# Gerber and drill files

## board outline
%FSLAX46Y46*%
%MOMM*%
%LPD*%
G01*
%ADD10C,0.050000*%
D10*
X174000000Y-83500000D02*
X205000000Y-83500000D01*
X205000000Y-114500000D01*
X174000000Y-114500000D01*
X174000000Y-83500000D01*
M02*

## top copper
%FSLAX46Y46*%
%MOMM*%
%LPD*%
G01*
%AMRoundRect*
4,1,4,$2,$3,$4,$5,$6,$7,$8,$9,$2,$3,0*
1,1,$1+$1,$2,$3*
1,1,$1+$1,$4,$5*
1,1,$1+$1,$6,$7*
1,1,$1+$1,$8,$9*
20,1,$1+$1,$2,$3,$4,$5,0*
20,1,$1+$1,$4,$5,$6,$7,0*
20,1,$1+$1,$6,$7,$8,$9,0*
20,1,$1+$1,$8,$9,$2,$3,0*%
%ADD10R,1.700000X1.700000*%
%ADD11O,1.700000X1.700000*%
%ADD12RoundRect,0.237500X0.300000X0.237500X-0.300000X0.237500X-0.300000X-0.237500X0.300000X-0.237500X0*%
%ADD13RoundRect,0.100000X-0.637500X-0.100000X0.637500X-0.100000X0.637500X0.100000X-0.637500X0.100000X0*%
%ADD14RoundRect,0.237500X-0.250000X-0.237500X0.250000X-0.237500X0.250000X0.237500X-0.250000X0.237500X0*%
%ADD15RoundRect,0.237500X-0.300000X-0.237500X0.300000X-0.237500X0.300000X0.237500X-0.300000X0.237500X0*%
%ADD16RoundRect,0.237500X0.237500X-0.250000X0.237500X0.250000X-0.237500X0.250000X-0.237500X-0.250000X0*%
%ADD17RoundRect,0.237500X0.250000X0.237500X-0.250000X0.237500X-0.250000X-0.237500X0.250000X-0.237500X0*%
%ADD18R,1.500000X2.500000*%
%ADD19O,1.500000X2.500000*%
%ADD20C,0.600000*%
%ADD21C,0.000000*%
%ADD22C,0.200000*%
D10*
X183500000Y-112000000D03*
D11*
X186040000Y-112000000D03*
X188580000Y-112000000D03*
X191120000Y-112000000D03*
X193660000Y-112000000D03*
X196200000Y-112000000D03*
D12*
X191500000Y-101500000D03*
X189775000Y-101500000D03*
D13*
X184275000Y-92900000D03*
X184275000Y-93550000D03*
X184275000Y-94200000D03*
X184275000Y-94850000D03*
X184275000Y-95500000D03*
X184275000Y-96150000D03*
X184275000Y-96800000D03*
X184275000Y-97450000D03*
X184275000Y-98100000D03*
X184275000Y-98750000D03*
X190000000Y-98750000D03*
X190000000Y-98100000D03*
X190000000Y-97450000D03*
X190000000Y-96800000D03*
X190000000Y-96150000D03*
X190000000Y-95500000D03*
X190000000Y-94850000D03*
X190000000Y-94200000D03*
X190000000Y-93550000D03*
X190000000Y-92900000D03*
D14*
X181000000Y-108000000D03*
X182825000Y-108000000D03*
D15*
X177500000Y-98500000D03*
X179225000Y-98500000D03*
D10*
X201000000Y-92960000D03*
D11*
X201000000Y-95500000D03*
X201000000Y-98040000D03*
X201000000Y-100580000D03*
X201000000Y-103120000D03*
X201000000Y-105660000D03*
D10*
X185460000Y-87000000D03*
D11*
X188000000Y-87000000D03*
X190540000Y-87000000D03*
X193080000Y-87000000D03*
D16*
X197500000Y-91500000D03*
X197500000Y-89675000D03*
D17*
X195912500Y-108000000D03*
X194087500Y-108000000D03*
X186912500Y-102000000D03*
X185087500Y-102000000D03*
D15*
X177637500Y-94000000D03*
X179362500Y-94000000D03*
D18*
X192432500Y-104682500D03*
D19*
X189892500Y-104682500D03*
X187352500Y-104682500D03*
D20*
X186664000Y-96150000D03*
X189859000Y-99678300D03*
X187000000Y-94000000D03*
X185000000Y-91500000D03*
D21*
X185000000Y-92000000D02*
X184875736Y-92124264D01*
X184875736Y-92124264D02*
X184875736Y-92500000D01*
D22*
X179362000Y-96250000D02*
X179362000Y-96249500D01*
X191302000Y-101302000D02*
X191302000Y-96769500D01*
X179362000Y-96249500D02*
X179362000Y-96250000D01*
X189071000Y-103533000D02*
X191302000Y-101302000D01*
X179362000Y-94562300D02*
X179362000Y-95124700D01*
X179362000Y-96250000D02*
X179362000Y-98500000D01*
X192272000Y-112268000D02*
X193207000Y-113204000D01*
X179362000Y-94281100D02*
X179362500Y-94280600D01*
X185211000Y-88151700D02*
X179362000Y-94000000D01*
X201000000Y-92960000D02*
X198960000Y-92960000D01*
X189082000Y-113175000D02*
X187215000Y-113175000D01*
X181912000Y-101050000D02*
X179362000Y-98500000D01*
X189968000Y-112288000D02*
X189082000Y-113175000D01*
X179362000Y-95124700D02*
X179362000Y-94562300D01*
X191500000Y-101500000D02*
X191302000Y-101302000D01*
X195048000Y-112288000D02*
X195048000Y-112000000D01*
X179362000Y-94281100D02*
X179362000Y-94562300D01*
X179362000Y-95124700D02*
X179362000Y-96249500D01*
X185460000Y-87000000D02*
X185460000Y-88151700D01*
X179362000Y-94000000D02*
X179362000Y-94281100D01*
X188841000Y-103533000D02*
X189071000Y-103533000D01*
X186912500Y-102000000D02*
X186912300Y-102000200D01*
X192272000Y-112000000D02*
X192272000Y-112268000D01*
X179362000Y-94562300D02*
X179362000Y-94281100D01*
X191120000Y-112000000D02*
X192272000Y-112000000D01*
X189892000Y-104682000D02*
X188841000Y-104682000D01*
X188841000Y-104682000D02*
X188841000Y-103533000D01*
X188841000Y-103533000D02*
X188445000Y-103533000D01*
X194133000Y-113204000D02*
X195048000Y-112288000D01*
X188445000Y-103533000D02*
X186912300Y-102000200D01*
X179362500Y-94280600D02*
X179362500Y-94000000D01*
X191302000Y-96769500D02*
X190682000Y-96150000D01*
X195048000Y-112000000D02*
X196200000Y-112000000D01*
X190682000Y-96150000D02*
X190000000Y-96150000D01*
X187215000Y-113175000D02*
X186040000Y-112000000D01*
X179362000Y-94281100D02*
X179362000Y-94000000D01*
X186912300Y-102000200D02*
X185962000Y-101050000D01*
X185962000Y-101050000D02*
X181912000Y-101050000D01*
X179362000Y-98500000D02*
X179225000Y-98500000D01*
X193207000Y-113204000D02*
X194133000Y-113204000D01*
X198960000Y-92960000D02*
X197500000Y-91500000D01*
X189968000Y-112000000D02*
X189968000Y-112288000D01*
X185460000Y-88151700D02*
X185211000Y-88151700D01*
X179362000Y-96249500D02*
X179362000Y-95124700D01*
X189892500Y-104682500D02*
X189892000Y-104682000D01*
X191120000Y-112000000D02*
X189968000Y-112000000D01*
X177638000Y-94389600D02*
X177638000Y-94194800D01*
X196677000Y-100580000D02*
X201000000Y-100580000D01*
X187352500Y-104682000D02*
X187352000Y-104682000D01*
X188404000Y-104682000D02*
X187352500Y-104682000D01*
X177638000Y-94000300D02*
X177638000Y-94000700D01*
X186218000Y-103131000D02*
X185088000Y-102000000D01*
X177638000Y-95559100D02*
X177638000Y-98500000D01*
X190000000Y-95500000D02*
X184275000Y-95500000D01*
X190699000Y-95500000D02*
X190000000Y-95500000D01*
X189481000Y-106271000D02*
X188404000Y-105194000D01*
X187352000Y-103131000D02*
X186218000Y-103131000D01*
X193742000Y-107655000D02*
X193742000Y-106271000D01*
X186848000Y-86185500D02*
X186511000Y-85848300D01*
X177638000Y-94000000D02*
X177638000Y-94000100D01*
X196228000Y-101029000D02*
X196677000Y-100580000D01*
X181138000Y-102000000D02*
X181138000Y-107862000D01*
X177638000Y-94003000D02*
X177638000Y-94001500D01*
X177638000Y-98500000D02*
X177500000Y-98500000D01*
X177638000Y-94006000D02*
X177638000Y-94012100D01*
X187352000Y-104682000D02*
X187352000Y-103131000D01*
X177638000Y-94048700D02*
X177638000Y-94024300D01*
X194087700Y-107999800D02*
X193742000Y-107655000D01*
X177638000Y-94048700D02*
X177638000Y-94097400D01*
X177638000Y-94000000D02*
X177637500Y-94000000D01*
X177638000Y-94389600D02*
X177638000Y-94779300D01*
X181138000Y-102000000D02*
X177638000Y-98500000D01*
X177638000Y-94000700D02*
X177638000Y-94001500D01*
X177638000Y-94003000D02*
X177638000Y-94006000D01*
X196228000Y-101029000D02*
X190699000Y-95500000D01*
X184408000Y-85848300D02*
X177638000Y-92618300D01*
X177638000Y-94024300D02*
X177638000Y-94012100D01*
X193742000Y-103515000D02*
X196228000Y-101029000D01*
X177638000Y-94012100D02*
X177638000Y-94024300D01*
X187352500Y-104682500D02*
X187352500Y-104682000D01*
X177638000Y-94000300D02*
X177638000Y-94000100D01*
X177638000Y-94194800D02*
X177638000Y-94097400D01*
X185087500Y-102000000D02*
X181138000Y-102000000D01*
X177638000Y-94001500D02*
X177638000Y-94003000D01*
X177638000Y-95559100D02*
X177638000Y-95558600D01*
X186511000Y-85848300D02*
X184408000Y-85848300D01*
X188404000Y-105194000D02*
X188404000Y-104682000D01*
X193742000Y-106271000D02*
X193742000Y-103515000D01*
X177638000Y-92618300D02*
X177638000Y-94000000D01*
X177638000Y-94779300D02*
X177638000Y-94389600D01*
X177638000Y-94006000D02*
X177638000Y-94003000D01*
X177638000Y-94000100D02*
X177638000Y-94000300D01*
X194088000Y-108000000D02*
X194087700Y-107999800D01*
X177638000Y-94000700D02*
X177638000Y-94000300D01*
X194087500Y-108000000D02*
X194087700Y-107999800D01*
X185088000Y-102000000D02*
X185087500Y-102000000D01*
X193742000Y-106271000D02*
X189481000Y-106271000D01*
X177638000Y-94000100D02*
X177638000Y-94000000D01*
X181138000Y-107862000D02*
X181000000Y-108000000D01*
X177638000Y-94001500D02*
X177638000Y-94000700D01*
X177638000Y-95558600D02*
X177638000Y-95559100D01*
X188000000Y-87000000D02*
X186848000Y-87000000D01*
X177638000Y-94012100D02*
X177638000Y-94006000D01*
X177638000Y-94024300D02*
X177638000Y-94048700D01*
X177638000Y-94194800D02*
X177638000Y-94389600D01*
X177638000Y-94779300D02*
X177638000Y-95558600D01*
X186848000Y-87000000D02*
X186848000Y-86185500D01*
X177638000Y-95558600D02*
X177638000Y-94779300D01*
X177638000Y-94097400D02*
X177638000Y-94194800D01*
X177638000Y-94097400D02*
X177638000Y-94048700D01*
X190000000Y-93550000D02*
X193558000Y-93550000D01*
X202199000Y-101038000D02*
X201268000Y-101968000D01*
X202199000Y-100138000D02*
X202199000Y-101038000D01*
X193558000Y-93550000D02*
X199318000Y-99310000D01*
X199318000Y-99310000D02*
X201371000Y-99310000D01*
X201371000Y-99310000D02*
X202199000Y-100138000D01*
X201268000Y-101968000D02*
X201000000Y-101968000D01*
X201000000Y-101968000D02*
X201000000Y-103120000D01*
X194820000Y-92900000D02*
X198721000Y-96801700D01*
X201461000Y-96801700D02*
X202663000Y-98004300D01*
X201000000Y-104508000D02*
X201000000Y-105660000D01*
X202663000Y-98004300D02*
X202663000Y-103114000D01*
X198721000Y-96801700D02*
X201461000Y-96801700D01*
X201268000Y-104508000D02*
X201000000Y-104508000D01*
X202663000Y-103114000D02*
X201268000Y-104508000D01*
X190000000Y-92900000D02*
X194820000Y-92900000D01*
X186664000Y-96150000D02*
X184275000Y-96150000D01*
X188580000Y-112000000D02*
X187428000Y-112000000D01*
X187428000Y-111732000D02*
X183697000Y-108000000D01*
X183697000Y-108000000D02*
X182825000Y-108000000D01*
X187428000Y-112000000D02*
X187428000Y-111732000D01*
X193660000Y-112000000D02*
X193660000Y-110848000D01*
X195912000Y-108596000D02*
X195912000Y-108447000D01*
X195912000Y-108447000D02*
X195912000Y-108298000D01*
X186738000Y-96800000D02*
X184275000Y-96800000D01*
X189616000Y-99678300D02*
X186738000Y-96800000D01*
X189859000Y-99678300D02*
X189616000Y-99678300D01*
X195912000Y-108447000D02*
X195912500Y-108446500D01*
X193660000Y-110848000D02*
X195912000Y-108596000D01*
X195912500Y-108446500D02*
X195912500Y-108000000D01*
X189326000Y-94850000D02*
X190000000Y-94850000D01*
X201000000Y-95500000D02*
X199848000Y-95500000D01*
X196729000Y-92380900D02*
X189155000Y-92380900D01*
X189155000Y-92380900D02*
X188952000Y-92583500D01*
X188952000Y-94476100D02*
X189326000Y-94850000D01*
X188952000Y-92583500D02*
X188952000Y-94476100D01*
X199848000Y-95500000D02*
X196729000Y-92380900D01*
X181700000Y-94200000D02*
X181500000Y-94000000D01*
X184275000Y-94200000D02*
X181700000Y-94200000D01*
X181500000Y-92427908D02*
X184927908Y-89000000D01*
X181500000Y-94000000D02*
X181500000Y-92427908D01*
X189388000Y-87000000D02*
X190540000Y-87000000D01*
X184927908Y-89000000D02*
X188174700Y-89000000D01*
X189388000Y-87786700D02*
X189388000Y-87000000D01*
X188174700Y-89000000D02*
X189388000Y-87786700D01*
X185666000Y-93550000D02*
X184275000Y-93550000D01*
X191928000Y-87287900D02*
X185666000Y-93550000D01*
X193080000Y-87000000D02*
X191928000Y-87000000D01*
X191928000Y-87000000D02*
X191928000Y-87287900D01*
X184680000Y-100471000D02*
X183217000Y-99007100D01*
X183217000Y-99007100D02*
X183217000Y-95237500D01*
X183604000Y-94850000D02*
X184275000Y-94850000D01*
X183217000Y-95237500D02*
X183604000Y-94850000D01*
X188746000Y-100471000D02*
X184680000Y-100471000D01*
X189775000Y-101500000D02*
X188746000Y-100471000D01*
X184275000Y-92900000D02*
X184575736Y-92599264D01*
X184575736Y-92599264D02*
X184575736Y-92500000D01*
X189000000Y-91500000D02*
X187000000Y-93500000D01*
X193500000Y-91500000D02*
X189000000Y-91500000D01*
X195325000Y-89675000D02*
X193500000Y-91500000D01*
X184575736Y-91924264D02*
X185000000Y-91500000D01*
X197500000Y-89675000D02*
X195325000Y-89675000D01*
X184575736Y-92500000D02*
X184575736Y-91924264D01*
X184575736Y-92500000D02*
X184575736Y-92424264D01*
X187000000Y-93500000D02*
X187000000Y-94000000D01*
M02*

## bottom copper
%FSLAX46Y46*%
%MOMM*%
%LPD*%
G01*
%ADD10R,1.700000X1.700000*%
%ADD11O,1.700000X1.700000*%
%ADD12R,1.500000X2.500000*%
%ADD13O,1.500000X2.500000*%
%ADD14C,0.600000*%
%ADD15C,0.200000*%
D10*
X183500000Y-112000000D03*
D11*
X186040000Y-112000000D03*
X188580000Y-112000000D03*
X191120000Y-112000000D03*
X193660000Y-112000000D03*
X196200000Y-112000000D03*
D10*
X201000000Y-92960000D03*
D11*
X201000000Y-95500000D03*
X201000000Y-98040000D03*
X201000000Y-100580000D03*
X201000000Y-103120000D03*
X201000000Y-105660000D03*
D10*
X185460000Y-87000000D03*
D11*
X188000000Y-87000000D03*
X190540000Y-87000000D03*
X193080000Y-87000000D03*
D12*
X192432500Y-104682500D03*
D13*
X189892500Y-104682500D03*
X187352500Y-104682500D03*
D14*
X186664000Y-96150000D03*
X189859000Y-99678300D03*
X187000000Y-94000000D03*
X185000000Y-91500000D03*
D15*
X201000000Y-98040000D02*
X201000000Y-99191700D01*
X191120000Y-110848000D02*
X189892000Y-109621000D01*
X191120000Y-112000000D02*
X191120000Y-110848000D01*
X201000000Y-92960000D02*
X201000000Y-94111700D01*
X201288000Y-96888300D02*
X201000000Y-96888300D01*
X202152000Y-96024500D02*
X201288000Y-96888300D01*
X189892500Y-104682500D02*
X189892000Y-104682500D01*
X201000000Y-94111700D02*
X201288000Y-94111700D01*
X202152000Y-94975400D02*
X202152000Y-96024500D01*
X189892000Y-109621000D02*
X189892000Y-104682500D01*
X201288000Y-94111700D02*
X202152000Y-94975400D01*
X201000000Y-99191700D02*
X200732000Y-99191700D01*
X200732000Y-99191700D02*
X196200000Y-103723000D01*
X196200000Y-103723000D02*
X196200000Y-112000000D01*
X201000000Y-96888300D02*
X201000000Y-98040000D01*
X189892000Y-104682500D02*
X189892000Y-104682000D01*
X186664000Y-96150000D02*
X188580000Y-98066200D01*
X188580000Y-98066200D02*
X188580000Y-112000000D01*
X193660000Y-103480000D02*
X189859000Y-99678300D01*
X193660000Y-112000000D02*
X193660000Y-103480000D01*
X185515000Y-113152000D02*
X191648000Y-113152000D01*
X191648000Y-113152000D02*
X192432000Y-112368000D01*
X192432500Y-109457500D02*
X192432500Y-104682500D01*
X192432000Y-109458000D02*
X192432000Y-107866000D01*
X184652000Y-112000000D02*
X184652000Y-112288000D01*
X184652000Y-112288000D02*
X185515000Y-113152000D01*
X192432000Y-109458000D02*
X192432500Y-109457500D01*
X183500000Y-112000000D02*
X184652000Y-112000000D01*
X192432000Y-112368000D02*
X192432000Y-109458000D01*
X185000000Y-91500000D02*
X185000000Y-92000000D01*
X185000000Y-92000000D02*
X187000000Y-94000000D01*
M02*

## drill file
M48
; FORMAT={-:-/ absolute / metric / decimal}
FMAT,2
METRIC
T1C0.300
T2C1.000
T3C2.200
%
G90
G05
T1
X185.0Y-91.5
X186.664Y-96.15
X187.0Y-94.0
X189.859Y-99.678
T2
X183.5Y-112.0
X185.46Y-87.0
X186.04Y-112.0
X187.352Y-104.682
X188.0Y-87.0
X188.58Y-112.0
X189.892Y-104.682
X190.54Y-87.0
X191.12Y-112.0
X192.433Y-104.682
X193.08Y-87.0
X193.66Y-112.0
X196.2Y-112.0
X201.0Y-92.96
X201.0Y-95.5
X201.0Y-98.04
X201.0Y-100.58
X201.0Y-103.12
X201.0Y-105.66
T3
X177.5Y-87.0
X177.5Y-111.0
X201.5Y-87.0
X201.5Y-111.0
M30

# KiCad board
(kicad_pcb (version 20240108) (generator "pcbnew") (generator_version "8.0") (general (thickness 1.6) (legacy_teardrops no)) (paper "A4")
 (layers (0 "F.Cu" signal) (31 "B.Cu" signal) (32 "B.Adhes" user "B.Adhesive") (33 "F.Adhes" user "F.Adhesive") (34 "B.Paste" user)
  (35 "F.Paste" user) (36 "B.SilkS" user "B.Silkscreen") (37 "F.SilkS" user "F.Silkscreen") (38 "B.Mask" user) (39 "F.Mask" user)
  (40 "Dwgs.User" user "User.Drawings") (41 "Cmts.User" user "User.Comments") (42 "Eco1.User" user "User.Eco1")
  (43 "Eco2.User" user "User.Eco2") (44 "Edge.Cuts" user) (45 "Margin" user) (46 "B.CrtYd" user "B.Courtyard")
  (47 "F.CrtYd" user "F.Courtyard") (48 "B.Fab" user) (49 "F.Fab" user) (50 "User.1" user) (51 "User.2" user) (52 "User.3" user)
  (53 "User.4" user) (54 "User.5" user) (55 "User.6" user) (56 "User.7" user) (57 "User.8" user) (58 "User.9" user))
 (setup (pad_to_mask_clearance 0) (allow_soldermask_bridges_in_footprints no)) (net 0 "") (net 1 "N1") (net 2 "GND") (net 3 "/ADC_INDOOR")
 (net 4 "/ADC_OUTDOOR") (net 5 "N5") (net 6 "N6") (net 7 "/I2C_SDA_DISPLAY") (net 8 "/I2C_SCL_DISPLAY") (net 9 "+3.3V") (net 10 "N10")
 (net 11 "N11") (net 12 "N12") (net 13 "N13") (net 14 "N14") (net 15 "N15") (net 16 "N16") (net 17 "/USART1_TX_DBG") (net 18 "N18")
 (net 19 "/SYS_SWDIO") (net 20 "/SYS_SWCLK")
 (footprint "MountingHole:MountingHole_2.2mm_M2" (layer "F.Cu") (at 201.5 111)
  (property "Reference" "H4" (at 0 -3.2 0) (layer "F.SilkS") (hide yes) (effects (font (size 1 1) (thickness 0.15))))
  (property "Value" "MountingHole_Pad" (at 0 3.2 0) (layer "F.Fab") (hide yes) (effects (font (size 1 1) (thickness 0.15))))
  (pad "" np_thru_hole circle (at 0 0) (size 2.2 2.2) (drill 2.2) (layers "*.Cu" "*.Mask")))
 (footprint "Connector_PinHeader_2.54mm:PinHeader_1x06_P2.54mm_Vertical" (layer "F.Cu") (at 183.5 112 90)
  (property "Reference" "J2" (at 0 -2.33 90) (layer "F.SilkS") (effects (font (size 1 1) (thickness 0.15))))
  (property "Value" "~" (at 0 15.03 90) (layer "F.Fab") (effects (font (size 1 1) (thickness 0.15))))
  (pad "1" thru_hole rect (at 0 0 90) (size 1.7 1.7) (drill 1) (layers "*.Cu" "*.Mask") (remove_unused_layers no) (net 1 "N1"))
  (pad "2" thru_hole oval (at 0 2.54 90) (size 1.7 1.7) (drill 1) (layers "*.Cu" "*.Mask") (remove_unused_layers no) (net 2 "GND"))
  (pad "3" thru_hole oval (at 0 5.08 90) (size 1.7 1.7) (drill 1) (layers "*.Cu" "*.Mask") (remove_unused_layers no) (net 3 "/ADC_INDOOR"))
  (pad "4" thru_hole oval (at 0 7.62 90) (size 1.7 1.7) (drill 1) (layers "*.Cu" "*.Mask") (remove_unused_layers no) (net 2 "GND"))
  (pad "5" thru_hole oval (at 0 10.16 90) (size 1.7 1.7) (drill 1) (layers "*.Cu" "*.Mask") (remove_unused_layers no) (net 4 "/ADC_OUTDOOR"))
  (pad "6" thru_hole oval (at 0 12.7 90) (size 1.7 1.7) (drill 1) (layers "*.Cu" "*.Mask") (remove_unused_layers no) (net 2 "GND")))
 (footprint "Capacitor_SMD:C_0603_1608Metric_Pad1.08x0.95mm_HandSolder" (layer "F.Cu") (at 190.6375 101.5 180)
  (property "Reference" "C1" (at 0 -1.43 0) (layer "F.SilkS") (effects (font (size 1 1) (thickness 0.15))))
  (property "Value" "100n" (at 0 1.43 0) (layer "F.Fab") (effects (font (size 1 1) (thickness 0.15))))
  (pad "1" smd roundrect (at -0.8625 0 180) (size 1.075 0.95) (layers "F.Cu" "F.Paste" "F.Mask") (roundrect_rratio 0.25) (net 2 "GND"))
  (pad "2" smd roundrect (at 0.8625 0 180) (size 1.075 0.95) (layers "F.Cu" "F.Paste" "F.Mask") (roundrect_rratio 0.25) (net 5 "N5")))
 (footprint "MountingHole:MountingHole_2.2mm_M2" (layer "F.Cu") (at 201.5 87)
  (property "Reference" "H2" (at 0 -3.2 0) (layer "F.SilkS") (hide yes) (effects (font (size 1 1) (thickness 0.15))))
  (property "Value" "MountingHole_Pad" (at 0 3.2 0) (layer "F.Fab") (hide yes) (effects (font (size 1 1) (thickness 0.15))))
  (pad "" np_thru_hole circle (at 0 0) (size 2.2 2.2) (drill 2.2) (layers "*.Cu" "*.Mask")))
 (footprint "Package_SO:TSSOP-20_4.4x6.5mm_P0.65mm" (layer "F.Cu") (at 187.1375 95.825)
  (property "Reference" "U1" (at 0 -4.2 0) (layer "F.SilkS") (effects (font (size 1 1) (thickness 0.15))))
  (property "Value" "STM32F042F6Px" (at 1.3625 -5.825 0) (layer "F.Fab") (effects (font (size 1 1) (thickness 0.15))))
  (pad "1" smd roundrect (at -2.8625 -2.925) (size 1.475 0.4) (layers "F.Cu" "F.Paste" "F.Mask") (roundrect_rratio 0.25) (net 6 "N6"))
  (pad "2" smd roundrect (at -2.8625 -2.275) (size 1.475 0.4) (layers "F.Cu" "F.Paste" "F.Mask") (roundrect_rratio 0.25)
   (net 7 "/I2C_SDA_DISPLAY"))
  (pad "3" smd roundrect (at -2.8625 -1.625) (size 1.475 0.4) (layers "F.Cu" "F.Paste" "F.Mask") (roundrect_rratio 0.25)
   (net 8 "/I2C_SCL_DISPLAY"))
  (pad "4" smd roundrect (at -2.8625 -0.975) (size 1.475 0.4) (layers "F.Cu" "F.Paste" "F.Mask") (roundrect_rratio 0.25) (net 5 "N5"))
  (pad "5" smd roundrect (at -2.8625 -0.325) (size 1.475 0.4) (layers "F.Cu" "F.Paste" "F.Mask") (roundrect_rratio 0.25) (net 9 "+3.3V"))
  (pad "6" smd roundrect (at -2.8625 0.325) (size 1.475 0.4) (layers "F.Cu" "F.Paste" "F.Mask") (roundrect_rratio 0.25)
   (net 3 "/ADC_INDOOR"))
  (pad "7" smd roundrect (at -2.8625 0.975) (size 1.475 0.4) (layers "F.Cu" "F.Paste" "F.Mask") (roundrect_rratio 0.25)
   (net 4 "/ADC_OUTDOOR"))
  (pad "8" smd roundrect (at -2.8625 1.625) (size 1.475 0.4) (layers "F.Cu" "F.Paste" "F.Mask") (roundrect_rratio 0.25) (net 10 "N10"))
  (pad "9" smd roundrect (at -2.8625 2.275) (size 1.475 0.4) (layers "F.Cu" "F.Paste" "F.Mask") (roundrect_rratio 0.25) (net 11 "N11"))
  (pad "10" smd roundrect (at -2.8625 2.925) (size 1.475 0.4) (layers "F.Cu" "F.Paste" "F.Mask") (roundrect_rratio 0.25) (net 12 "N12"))
  (pad "11" smd roundrect (at 2.8625 2.925) (size 1.475 0.4) (layers "F.Cu" "F.Paste" "F.Mask") (roundrect_rratio 0.25) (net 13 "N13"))
  (pad "12" smd roundrect (at 2.8625 2.275) (size 1.475 0.4) (layers "F.Cu" "F.Paste" "F.Mask") (roundrect_rratio 0.25) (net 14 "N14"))
  (pad "13" smd roundrect (at 2.8625 1.625) (size 1.475 0.4) (layers "F.Cu" "F.Paste" "F.Mask") (roundrect_rratio 0.25) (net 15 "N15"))
  (pad "14" smd roundrect (at 2.8625 0.975) (size 1.475 0.4) (layers "F.Cu" "F.Paste" "F.Mask") (roundrect_rratio 0.25) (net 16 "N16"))
  (pad "15" smd roundrect (at 2.8625 0.325) (size 1.475 0.4) (layers "F.Cu" "F.Paste" "F.Mask") (roundrect_rratio 0.25) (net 2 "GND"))
  (pad "16" smd roundrect (at 2.8625 -0.325) (size 1.475 0.4) (layers "F.Cu" "F.Paste" "F.Mask") (roundrect_rratio 0.25) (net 9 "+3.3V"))
  (pad "17" smd roundrect (at 2.8625 -0.975) (size 1.475 0.4) (layers "F.Cu" "F.Paste" "F.Mask") (roundrect_rratio 0.25)
   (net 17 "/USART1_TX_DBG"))
  (pad "18" smd roundrect (at 2.8625 -1.625) (size 1.475 0.4) (layers "F.Cu" "F.Paste" "F.Mask") (roundrect_rratio 0.25) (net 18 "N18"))
  (pad "19" smd roundrect (at 2.8625 -2.275) (size 1.475 0.4) (layers "F.Cu" "F.Paste" "F.Mask") (roundrect_rratio 0.25)
   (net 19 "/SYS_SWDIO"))
  (pad "20" smd roundrect (at 2.8625 -2.925) (size 1.475 0.4) (layers "F.Cu" "F.Paste" "F.Mask") (roundrect_rratio 0.25)
   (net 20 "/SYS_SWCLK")))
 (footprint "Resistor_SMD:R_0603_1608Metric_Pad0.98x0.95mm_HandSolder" (layer "F.Cu") (at 181.9125 108)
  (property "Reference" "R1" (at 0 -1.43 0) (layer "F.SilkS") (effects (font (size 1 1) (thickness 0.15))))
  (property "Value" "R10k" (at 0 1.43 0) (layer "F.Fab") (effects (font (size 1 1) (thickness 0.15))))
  (pad "1" smd roundrect (at -0.9125 0) (size 0.975 0.95) (layers "F.Cu" "F.Paste" "F.Mask") (roundrect_rratio 0.25) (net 9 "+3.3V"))
  (pad "2" smd roundrect (at 0.9125 0) (size 0.975 0.95) (layers "F.Cu" "F.Paste" "F.Mask") (roundrect_rratio 0.25) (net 3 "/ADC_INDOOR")))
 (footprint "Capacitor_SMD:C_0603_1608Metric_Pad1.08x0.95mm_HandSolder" (layer "F.Cu") (at 178.3625 98.5)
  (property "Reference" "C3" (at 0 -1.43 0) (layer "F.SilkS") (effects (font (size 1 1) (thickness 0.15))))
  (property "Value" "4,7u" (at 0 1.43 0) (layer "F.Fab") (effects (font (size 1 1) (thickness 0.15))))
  (pad "1" smd roundrect (at -0.8625 0) (size 1.075 0.95) (layers "F.Cu" "F.Paste" "F.Mask") (roundrect_rratio 0.25) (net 9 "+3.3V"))
  (pad "2" smd roundrect (at 0.8625 0) (size 1.075 0.95) (layers "F.Cu" "F.Paste" "F.Mask") (roundrect_rratio 0.25) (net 2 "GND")))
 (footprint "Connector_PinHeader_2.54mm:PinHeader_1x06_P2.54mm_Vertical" (layer "F.Cu") (at 201 92.96)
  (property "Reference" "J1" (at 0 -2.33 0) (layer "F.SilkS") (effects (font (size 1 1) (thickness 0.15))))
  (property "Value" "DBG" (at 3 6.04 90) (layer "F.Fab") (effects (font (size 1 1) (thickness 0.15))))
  (pad "1" thru_hole rect (at 0 0) (size 1.7 1.7) (drill 1) (layers "*.Cu" "*.Mask") (remove_unused_layers no) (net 2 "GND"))
  (pad "2" thru_hole oval (at 0 2.54) (size 1.7 1.7) (drill 1) (layers "*.Cu" "*.Mask") (remove_unused_layers no) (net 17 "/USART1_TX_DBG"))
  (pad "3" thru_hole oval (at 0 5.08) (size 1.7 1.7) (drill 1) (layers "*.Cu" "*.Mask") (remove_unused_layers no) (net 2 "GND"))
  (pad "4" thru_hole oval (at 0 7.62) (size 1.7 1.7) (drill 1) (layers "*.Cu" "*.Mask") (remove_unused_layers no) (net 9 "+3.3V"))
  (pad "5" thru_hole oval (at 0 10.16) (size 1.7 1.7) (drill 1) (layers "*.Cu" "*.Mask") (remove_unused_layers no) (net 19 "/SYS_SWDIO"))
  (pad "6" thru_hole oval (at 0 12.7) (size 1.7 1.7) (drill 1) (layers "*.Cu" "*.Mask") (remove_unused_layers no) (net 20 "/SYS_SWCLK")))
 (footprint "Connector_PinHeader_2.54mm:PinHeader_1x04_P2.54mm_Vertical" (layer "F.Cu") (at 185.46 87 90)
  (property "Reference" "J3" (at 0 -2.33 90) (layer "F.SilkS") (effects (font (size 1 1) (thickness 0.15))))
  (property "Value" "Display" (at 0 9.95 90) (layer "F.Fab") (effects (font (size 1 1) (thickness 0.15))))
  (pad "1" thru_hole rect (at 0 0 90) (size 1.7 1.7) (drill 1) (layers "*.Cu" "*.Mask") (remove_unused_layers no) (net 2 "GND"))
  (pad "2" thru_hole oval (at 0 2.54 90) (size 1.7 1.7) (drill 1) (layers "*.Cu" "*.Mask") (remove_unused_layers no) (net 9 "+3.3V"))
  (pad "3" thru_hole oval (at 0 5.08 90) (size 1.7 1.7) (drill 1) (layers "*.Cu" "*.Mask") (remove_unused_layers no)
   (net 8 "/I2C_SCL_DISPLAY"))
  (pad "4" thru_hole oval (at 0 7.62 90) (size 1.7 1.7) (drill 1) (layers "*.Cu" "*.Mask") (remove_unused_layers no)
   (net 7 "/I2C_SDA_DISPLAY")))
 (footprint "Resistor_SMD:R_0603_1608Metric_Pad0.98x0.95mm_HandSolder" (layer "F.Cu") (at 197.5 90.5875 90)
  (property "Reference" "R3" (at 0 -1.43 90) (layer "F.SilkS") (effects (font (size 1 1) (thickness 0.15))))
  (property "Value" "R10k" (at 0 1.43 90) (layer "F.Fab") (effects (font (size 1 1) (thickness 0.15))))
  (pad "1" smd roundrect (at -0.9125 0 90) (size 0.975 0.95) (layers "F.Cu" "F.Paste" "F.Mask") (roundrect_rratio 0.25) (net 2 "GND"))
  (pad "2" smd roundrect (at 0.9125 0 90) (size 0.975 0.95) (layers "F.Cu" "F.Paste" "F.Mask") (roundrect_rratio 0.25) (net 6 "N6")))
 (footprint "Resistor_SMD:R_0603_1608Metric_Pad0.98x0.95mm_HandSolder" (layer "F.Cu") (at 195 108 180)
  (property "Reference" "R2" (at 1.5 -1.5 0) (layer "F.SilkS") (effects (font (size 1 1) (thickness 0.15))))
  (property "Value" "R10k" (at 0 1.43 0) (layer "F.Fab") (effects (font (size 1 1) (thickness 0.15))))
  (pad "1" smd roundrect (at -0.9125 0 180) (size 0.975 0.95) (layers "F.Cu" "F.Paste" "F.Mask") (roundrect_rratio 0.25)
   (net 4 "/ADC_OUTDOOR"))
  (pad "2" smd roundrect (at 0.9125 0 180) (size 0.975 0.95) (layers "F.Cu" "F.Paste" "F.Mask") (roundrect_rratio 0.25) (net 9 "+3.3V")))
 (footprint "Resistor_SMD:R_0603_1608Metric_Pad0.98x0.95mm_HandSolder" (layer "F.Cu") (at 186 102 180)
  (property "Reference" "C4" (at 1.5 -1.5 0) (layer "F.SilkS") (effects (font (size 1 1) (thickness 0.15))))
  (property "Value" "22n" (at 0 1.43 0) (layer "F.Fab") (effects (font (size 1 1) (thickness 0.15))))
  (pad "1" smd roundrect (at -0.9125 0 180) (size 0.975 0.95) (layers "F.Cu" "F.Paste" "F.Mask") (roundrect_rratio 0.25) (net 2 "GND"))
  (pad "2" smd roundrect (at 0.9125 0 180) (size 0.975 0.95) (layers "F.Cu" "F.Paste" "F.Mask") (roundrect_rratio 0.25) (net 9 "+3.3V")))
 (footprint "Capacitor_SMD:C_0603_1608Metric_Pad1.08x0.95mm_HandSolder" (layer "F.Cu") (at 178.5 94)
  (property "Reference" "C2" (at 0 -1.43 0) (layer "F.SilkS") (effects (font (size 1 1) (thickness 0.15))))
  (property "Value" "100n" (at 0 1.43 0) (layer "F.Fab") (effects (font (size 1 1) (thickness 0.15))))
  (pad "1" smd roundrect (at -0.8625 0) (size 1.075 0.95) (layers "F.Cu" "F.Paste" "F.Mask") (roundrect_rratio 0.25) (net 9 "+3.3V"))
  (pad "2" smd roundrect (at 0.8625 0) (size 1.075 0.95) (layers "F.Cu" "F.Paste" "F.Mask") (roundrect_rratio 0.25) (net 2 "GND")))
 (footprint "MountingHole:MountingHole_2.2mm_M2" (layer "F.Cu") (at 177.5 87)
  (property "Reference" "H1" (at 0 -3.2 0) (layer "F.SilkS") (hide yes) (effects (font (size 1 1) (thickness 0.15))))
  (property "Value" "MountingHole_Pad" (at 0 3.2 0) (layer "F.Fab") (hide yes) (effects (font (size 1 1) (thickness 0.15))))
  (pad "" np_thru_hole circle (at 0 0) (size 2.2 2.2) (drill 2.2) (layers "*.Cu" "*.Mask")))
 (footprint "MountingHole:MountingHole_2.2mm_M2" (layer "F.Cu") (at 177.5 111)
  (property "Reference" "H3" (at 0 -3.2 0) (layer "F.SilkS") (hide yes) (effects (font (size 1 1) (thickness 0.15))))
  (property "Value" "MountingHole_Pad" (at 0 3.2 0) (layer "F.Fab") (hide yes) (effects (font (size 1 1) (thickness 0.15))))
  (pad "" np_thru_hole circle (at 0 0) (size 2.2 2.2) (drill 2.2) (layers "*.Cu" "*.Mask")))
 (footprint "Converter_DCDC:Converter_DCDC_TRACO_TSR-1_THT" (layer "B.Cu") (at 192.4325 104.6825 180)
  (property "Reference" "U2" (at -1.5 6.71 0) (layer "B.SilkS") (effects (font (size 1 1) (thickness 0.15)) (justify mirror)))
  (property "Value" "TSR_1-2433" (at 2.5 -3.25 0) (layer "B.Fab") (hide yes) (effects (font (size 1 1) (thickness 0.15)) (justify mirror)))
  (pad "1" thru_hole rect (at 0 0 180) (size 1.5 2.5) (drill 1) (layers "*.Cu" "*.Mask") (remove_unused_layers no) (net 1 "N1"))
  (pad "2" thru_hole oval (at 2.54 0 180) (size 1.5 2.5) (drill 1) (layers "*.Cu" "*.Mask") (remove_unused_layers no) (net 2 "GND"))
  (pad "3" thru_hole oval (at 5.08 0 180) (size 1.5 2.5) (drill 1) (layers "*.Cu" "*.Mask") (remove_unused_layers no) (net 9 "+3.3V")))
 (gr_rect (start 174 83.5) (end 205 114.5) (stroke (width 0.05) (type default)) (fill none) (layer "Edge.Cuts"))
 (segment (start 185 92) (end 184.875736 92.124264) (width 0) (layer "F.Cu") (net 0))
 (segment (start 184.875736 92.124264) (end 184.875736 92.5) (width 0) (layer "F.Cu") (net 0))
 (segment (start 179.362 96.25) (end 179.362 96.2495) (width 0.2) (layer "F.Cu") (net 2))
 (segment (start 191.302 101.302) (end 191.302 96.7695) (width 0.2) (layer "F.Cu") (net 2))
 (segment (start 179.362 96.2495) (end 179.362 96.25) (width 0.2) (layer "F.Cu") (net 2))
 (segment (start 189.071 103.533) (end 191.302 101.302) (width 0.2) (layer "F.Cu") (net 2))
 (segment (start 179.362 94.5623) (end 179.362 95.1247) (width 0.2) (layer "F.Cu") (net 2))
 (segment (start 179.362 96.25) (end 179.362 98.5) (width 0.2) (layer "F.Cu") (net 2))
 (segment (start 192.272 112.268) (end 193.207 113.204) (width 0.2) (layer "F.Cu") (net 2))
 (segment (start 179.362 94.2811) (end 179.3625 94.2806) (width 0.2) (layer "F.Cu") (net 2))
 (segment (start 185.211 88.1517) (end 179.362 94) (width 0.2) (layer "F.Cu") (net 2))
 (segment (start 201 92.96) (end 198.96 92.96) (width 0.2) (layer "F.Cu") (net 2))
 (segment (start 189.082 113.175) (end 187.215 113.175) (width 0.2) (layer "F.Cu") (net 2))
 (segment (start 181.912 101.05) (end 179.362 98.5) (width 0.2) (layer "F.Cu") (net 2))
 (segment (start 189.968 112.288) (end 189.082 113.175) (width 0.2) (layer "F.Cu") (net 2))
 (segment (start 179.362 95.1247) (end 179.362 94.5623) (width 0.2) (layer "F.Cu") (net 2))
 (segment (start 191.5 101.5) (end 191.302 101.302) (width 0.2) (layer "F.Cu") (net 2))
 (segment (start 195.048 112.288) (end 195.048 112) (width 0.2) (layer "F.Cu") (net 2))
 (segment (start 179.362 94.2811) (end 179.362 94.5623) (width 0.2) (layer "F.Cu") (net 2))
 (segment (start 179.362 95.1247) (end 179.362 96.2495) (width 0.2) (layer "F.Cu") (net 2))
 (segment (start 185.46 87) (end 185.46 88.1517) (width 0.2) (layer "F.Cu") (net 2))
 (segment (start 179.362 94) (end 179.362 94.2811) (width 0.2) (layer "F.Cu") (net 2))
 (segment (start 188.841 103.533) (end 189.071 103.533) (width 0.2) (layer "F.Cu") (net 2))
 (segment (start 186.9125 102) (end 186.9123 102.0002) (width 0.2) (layer "F.Cu") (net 2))
 (segment (start 192.272 112) (end 192.272 112.268) (width 0.2) (layer "F.Cu") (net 2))
 (segment (start 179.362 94.5623) (end 179.362 94.2811) (width 0.2) (layer "F.Cu") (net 2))
 (segment (start 191.12 112) (end 192.272 112) (width 0.2) (layer "F.Cu") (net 2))
 (segment (start 189.892 104.682) (end 188.841 104.682) (width 0.2) (layer "F.Cu") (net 2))
 (segment (start 188.841 104.682) (end 188.841 103.533) (width 0.2) (layer "F.Cu") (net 2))
 (segment (start 188.841 103.533) (end 188.445 103.533) (width 0.2) (layer "F.Cu") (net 2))
 (segment (start 194.133 113.204) (end 195.048 112.288) (width 0.2) (layer "F.Cu") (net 2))
 (segment (start 188.445 103.533) (end 186.9123 102.0002) (width 0.2) (layer "F.Cu") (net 2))
 (segment (start 179.3625 94.2806) (end 179.3625 94) (width 0.2) (layer "F.Cu") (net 2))
 (segment (start 191.302 96.7695) (end 190.682 96.15) (width 0.2) (layer "F.Cu") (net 2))
 (segment (start 195.048 112) (end 196.2 112) (width 0.2) (layer "F.Cu") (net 2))
 (segment (start 190.682 96.15) (end 190 96.15) (width 0.2) (layer "F.Cu") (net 2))
 (segment (start 187.215 113.175) (end 186.04 112) (width 0.2) (layer "F.Cu") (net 2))
 (segment (start 179.362 94.2811) (end 179.362 94) (width 0.2) (layer "F.Cu") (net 2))
 (segment (start 186.9123 102.0002) (end 185.962 101.05) (width 0.2) (layer "F.Cu") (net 2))
 (segment (start 185.962 101.05) (end 181.912 101.05) (width 0.2) (layer "F.Cu") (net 2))
 (segment (start 179.362 98.5) (end 179.225 98.5) (width 0.2) (layer "F.Cu") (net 2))
 (segment (start 193.207 113.204) (end 194.133 113.204) (width 0.2) (layer "F.Cu") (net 2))
 (segment (start 198.96 92.96) (end 197.5 91.5) (width 0.2) (layer "F.Cu") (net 2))
 (segment (start 189.968 112) (end 189.968 112.288) (width 0.2) (layer "F.Cu") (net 2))
 (segment (start 185.46 88.1517) (end 185.211 88.1517) (width 0.2) (layer "F.Cu") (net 2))
 (segment (start 179.362 96.2495) (end 179.362 95.1247) (width 0.2) (layer "F.Cu") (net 2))
 (segment (start 189.8925 104.6825) (end 189.892 104.682) (width 0.2) (layer "F.Cu") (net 2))
 (segment (start 191.12 112) (end 189.968 112) (width 0.2) (layer "F.Cu") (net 2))
 (segment (start 201 98.04) (end 201 99.1917) (width 0.2) (layer "B.Cu") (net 2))
 (segment (start 191.12 110.848) (end 189.892 109.621) (width 0.2) (layer "B.Cu") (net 2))
 (segment (start 191.12 112) (end 191.12 110.848) (width 0.2) (layer "B.Cu") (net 2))
 (segment (start 201 92.96) (end 201 94.1117) (width 0.2) (layer "B.Cu") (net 2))
 (segment (start 201.288 96.8883) (end 201 96.8883) (width 0.2) (layer "B.Cu") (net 2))
 (segment (start 202.152 96.0245) (end 201.288 96.8883) (width 0.2) (layer "B.Cu") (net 2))
 (segment (start 189.8925 104.6825) (end 189.892 104.6825) (width 0.2) (layer "B.Cu") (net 2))
 (segment (start 201 94.1117) (end 201.288 94.1117) (width 0.2) (layer "B.Cu") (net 2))
 (segment (start 202.152 94.9754) (end 202.152 96.0245) (width 0.2) (layer "B.Cu") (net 2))
 (segment (start 189.892 109.621) (end 189.892 104.6825) (width 0.2) (layer "B.Cu") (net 2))
 (segment (start 201.288 94.1117) (end 202.152 94.9754) (width 0.2) (layer "B.Cu") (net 2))
 (segment (start 201 99.1917) (end 200.732 99.1917) (width 0.2) (layer "B.Cu") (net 2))
 (segment (start 200.732 99.1917) (end 196.2 103.723) (width 0.2) (layer "B.Cu") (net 2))
 (segment (start 196.2 103.723) (end 196.2 112) (width 0.2) (layer "B.Cu") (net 2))
 (segment (start 201 96.8883) (end 201 98.04) (width 0.2) (layer "B.Cu") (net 2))
 (segment (start 189.892 104.6825) (end 189.892 104.682) (width 0.2) (layer "B.Cu") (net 2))
 (segment (start 177.638 94.3896) (end 177.638 94.1948) (width 0.2) (layer "F.Cu") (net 9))
 (segment (start 196.677 100.58) (end 201 100.58) (width 0.2) (layer "F.Cu") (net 9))
 (segment (start 187.3525 104.682) (end 187.352 104.682) (width 0.2) (layer "F.Cu") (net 9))
 (segment (start 188.404 104.682) (end 187.3525 104.682) (width 0.2) (layer "F.Cu") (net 9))
 (segment (start 177.638 94.0003) (end 177.638 94.0007) (width 0.2) (layer "F.Cu") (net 9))
 (segment (start 186.218 103.131) (end 185.088 102) (width 0.2) (layer "F.Cu") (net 9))
 (segment (start 177.638 95.5591) (end 177.638 98.5) (width 0.2) (layer "F.Cu") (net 9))
 (segment (start 190 95.5) (end 184.275 95.5) (width 0.2) (layer "F.Cu") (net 9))
 (segment (start 190.699 95.5) (end 190 95.5) (width 0.2) (layer "F.Cu") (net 9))
 (segment (start 189.481 106.271) (end 188.404 105.194) (width 0.2) (layer "F.Cu") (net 9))
 (segment (start 187.352 103.131) (end 186.218 103.131) (width 0.2) (layer "F.Cu") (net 9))
 (segment (start 193.742 107.655) (end 193.742 106.271) (width 0.2) (layer "F.Cu") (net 9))
 (segment (start 186.848 86.1855) (end 186.511 85.8483) (width 0.2) (layer "F.Cu") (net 9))
 (segment (start 177.638 94) (end 177.638 94.0001) (width 0.2) (layer "F.Cu") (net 9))
 (segment (start 196.228 101.029) (end 196.677 100.58) (width 0.2) (layer "F.Cu") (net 9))
 (segment (start 181.138 102) (end 181.138 107.862) (width 0.2) (layer "F.Cu") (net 9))
 (segment (start 177.638 94.003) (end 177.638 94.0015) (width 0.2) (layer "F.Cu") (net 9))
 (segment (start 177.638 98.5) (end 177.5 98.5) (width 0.2) (layer "F.Cu") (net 9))
 (segment (start 177.638 94.006) (end 177.638 94.0121) (width 0.2) (layer "F.Cu") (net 9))
 (segment (start 187.352 104.682) (end 187.352 103.131) (width 0.2) (layer "F.Cu") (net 9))
 (segment (start 177.638 94.0487) (end 177.638 94.0243) (width 0.2) (layer "F.Cu") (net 9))
 (segment (start 194.0877 107.9998) (end 193.742 107.655) (width 0.2) (layer "F.Cu") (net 9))
 (segment (start 177.638 94.0487) (end 177.638 94.0974) (width 0.2) (layer "F.Cu") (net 9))
 (segment (start 177.638 94) (end 177.6375 94) (width 0.2) (layer "F.Cu") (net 9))
 (segment (start 177.638 94.3896) (end 177.638 94.7793) (width 0.2) (layer "F.Cu") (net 9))
 (segment (start 181.138 102) (end 177.638 98.5) (width 0.2) (layer "F.Cu") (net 9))
 (segment (start 177.638 94.0007) (end 177.638 94.0015) (width 0.2) (layer "F.Cu") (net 9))
 (segment (start 177.638 94.003) (end 177.638 94.006) (width 0.2) (layer "F.Cu") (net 9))
 (segment (start 196.228 101.029) (end 190.699 95.5) (width 0.2) (layer "F.Cu") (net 9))
 (segment (start 184.408 85.8483) (end 177.638 92.6183) (width 0.2) (layer "F.Cu") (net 9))
 (segment (start 177.638 94.0243) (end 177.638 94.0121) (width 0.2) (layer "F.Cu") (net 9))
 (segment (start 193.742 103.515) (end 196.228 101.029) (width 0.2) (layer "F.Cu") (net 9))
 (segment (start 177.638 94.0121) (end 177.638 94.0243) (width 0.2) (layer "F.Cu") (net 9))
 (segment (start 187.3525 104.6825) (end 187.3525 104.682) (width 0.2) (layer "F.Cu") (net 9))
 (segment (start 177.638 94.0003) (end 177.638 94.0001) (width 0.2) (layer "F.Cu") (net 9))
 (segment (start 177.638 94.1948) (end 177.638 94.0974) (width 0.2) (layer "F.Cu") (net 9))
 (segment (start 185.0875 102) (end 181.138 102) (width 0.2) (layer "F.Cu") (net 9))
 (segment (start 177.638 94.0015) (end 177.638 94.003) (width 0.2) (layer "F.Cu") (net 9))
 (segment (start 177.638 95.5591) (end 177.638 95.5586) (width 0.2) (layer "F.Cu") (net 9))
 (segment (start 186.511 85.8483) (end 184.408 85.8483) (width 0.2) (layer "F.Cu") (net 9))
 (segment (start 188.404 105.194) (end 188.404 104.682) (width 0.2) (layer "F.Cu") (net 9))
 (segment (start 193.742 106.271) (end 193.742 103.515) (width 0.2) (layer "F.Cu") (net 9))
 (segment (start 177.638 92.6183) (end 177.638 94) (width 0.2) (layer "F.Cu") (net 9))
 (segment (start 177.638 94.7793) (end 177.638 94.3896) (width 0.2) (layer "F.Cu") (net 9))
 (segment (start 177.638 94.006) (end 177.638 94.003) (width 0.2) (layer "F.Cu") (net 9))
 (segment (start 177.638 94.0001) (end 177.638 94.0003) (width 0.2) (layer "F.Cu") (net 9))
 (segment (start 194.088 108) (end 194.0877 107.9998) (width 0.2) (layer "F.Cu") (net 9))
 (segment (start 177.638 94.0007) (end 177.638 94.0003) (width 0.2) (layer "F.Cu") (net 9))
 (segment (start 194.0875 108) (end 194.0877 107.9998) (width 0.2) (layer "F.Cu") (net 9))
 (segment (start 185.088 102) (end 185.0875 102) (width 0.2) (layer "F.Cu") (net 9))
 (segment (start 193.742 106.271) (end 189.481 106.271) (width 0.2) (layer "F.Cu") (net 9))
 (segment (start 177.638 94.0001) (end 177.638 94) (width 0.2) (layer "F.Cu") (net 9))
 (segment (start 181.138 107.862) (end 181 108) (width 0.2) (layer "F.Cu") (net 9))
 (segment (start 177.638 94.0015) (end 177.638 94.0007) (width 0.2) (layer "F.Cu") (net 9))
 (segment (start 177.638 95.5586) (end 177.638 95.5591) (width 0.2) (layer "F.Cu") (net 9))
 (segment (start 188 87) (end 186.848 87) (width 0.2) (layer "F.Cu") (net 9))
 (segment (start 177.638 94.0121) (end 177.638 94.006) (width 0.2) (layer "F.Cu") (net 9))
 (segment (start 177.638 94.0243) (end 177.638 94.0487) (width 0.2) (layer "F.Cu") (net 9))
 (segment (start 177.638 94.1948) (end 177.638 94.3896) (width 0.2) (layer "F.Cu") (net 9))
 (segment (start 177.638 94.7793) (end 177.638 95.5586) (width 0.2) (layer "F.Cu") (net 9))
 (segment (start 186.848 87) (end 186.848 86.1855) (width 0.2) (layer "F.Cu") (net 9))
 (segment (start 177.638 95.5586) (end 177.638 94.7793) (width 0.2) (layer "F.Cu") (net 9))
 (segment (start 177.638 94.0974) (end 177.638 94.1948) (width 0.2) (layer "F.Cu") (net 9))
 (segment (start 177.638 94.0974) (end 177.638 94.0487) (width 0.2) (layer "F.Cu") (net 9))
 (segment (start 190 93.55) (end 193.558 93.55) (width 0.2) (layer "F.Cu") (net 19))
 (segment (start 202.199 101.038) (end 201.268 101.968) (width 0.2) (layer "F.Cu") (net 19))
 (segment (start 202.199 100.138) (end 202.199 101.038) (width 0.2) (layer "F.Cu") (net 19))
 (segment (start 193.558 93.55) (end 199.318 99.31) (width 0.2) (layer "F.Cu") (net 19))
 (segment (start 199.318 99.31) (end 201.371 99.31) (width 0.2) (layer "F.Cu") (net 19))
 (segment (start 201.371 99.31) (end 202.199 100.138) (width 0.2) (layer "F.Cu") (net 19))
 (segment (start 201.268 101.968) (end 201 101.968) (width 0.2) (layer "F.Cu") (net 19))
 (segment (start 201 101.968) (end 201 103.12) (width 0.2) (layer "F.Cu") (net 19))
 (segment (start 194.82 92.9) (end 198.721 96.8017) (width 0.2) (layer "F.Cu") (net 20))
 (segment (start 201.461 96.8017) (end 202.663 98.0043) (width 0.2) (layer "F.Cu") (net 20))
 (segment (start 201 104.508) (end 201 105.66) (width 0.2) (layer "F.Cu") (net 20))
 (segment (start 202.663 98.0043) (end 202.663 103.114) (width 0.2) (layer "F.Cu") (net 20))
 (segment (start 198.721 96.8017) (end 201.461 96.8017) (width 0.2) (layer "F.Cu") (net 20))
 (segment (start 201.268 104.508) (end 201 104.508) (width 0.2) (layer "F.Cu") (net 20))
 (segment (start 202.663 103.114) (end 201.268 104.508) (width 0.2) (layer "F.Cu") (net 20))
 (segment (start 190 92.9) (end 194.82 92.9) (width 0.2) (layer "F.Cu") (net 20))
 (segment (start 186.664 96.15) (end 184.275 96.15) (width 0.2) (layer "F.Cu") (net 3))
 (segment (start 188.58 112) (end 187.428 112) (width 0.2) (layer "F.Cu") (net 3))
 (segment (start 187.428 111.732) (end 183.697 108) (width 0.2) (layer "F.Cu") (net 3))
 (segment (start 183.697 108) (end 182.825 108) (width 0.2) (layer "F.Cu") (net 3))
 (segment (start 187.428 112) (end 187.428 111.732) (width 0.2) (layer "F.Cu") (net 3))
 (via (at 186.664 96.15) (size 0.6) (drill 0.3) (layers "F.Cu" "B.Cu") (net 3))
 (segment (start 186.664 96.15) (end 188.58 98.0662) (width 0.2) (layer "B.Cu") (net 3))
 (segment (start 188.58 98.0662) (end 188.58 112) (width 0.2) (layer "B.Cu") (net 3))
 (segment (start 193.66 112) (end 193.66 110.848) (width 0.2) (layer "F.Cu") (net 4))
 (segment (start 195.912 108.596) (end 195.912 108.447) (width 0.2) (layer "F.Cu") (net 4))
 (segment (start 195.912 108.447) (end 195.912 108.298) (width 0.2) (layer "F.Cu") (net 4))
 (segment (start 186.738 96.8) (end 184.275 96.8) (width 0.2) (layer "F.Cu") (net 4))
 (segment (start 189.616 99.6783) (end 186.738 96.8) (width 0.2) (layer "F.Cu") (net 4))
 (segment (start 189.859 99.6783) (end 189.616 99.6783) (width 0.2) (layer "F.Cu") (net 4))
 (segment (start 195.912 108.447) (end 195.9125 108.4465) (width 0.2) (layer "F.Cu") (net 4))
 (segment (start 193.66 110.848) (end 195.912 108.596) (width 0.2) (layer "F.Cu") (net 4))
 (segment (start 195.9125 108.4465) (end 195.9125 108) (width 0.2) (layer "F.Cu") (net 4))
 (via (at 189.859 99.6783) (size 0.6) (drill 0.3) (layers "F.Cu" "B.Cu") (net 4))
 (segment (start 193.66 103.48) (end 189.859 99.6783) (width 0.2) (layer "B.Cu") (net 4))
 (segment (start 193.66 112) (end 193.66 103.48) (width 0.2) (layer "B.Cu") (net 4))
 (segment (start 189.326 94.85) (end 190 94.85) (width 0.2) (layer "F.Cu") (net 17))
 (segment (start 201 95.5) (end 199.848 95.5) (width 0.2) (layer "F.Cu") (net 17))
 (segment (start 196.729 92.3809) (end 189.155 92.3809) (width 0.2) (layer "F.Cu") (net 17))
 (segment (start 189.155 92.3809) (end 188.952 92.5835) (width 0.2) (layer "F.Cu") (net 17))
 (segment (start 188.952 94.4761) (end 189.326 94.85) (width 0.2) (layer "F.Cu") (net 17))
 (segment (start 188.952 92.5835) (end 188.952 94.4761) (width 0.2) (layer "F.Cu") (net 17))
 (segment (start 199.848 95.5) (end 196.729 92.3809) (width 0.2) (layer "F.Cu") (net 17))
 (segment (start 181.7 94.2) (end 181.5 94) (width 0.2) (layer "F.Cu") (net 8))
 (segment (start 184.275 94.2) (end 181.7 94.2) (width 0.2) (layer "F.Cu") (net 8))
 (segment (start 181.5 92.427908) (end 184.927908 89) (width 0.2) (layer "F.Cu") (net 8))
 (segment (start 181.5 94) (end 181.5 92.427908) (width 0.2) (layer "F.Cu") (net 8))
 (segment (start 189.388 87) (end 190.54 87) (width 0.2) (layer "F.Cu") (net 8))
 (segment (start 184.927908 89) (end 188.1747 89) (width 0.2) (layer "F.Cu") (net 8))
 (segment (start 189.388 87.7867) (end 189.388 87) (width 0.2) (layer "F.Cu") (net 8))
 (segment (start 188.1747 89) (end 189.388 87.7867) (width 0.2) (layer "F.Cu") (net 8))
 (segment (start 185.666 93.55) (end 184.275 93.55) (width 0.2) (layer "F.Cu") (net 7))
 (segment (start 191.928 87.2879) (end 185.666 93.55) (width 0.2) (layer "F.Cu") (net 7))
 (segment (start 193.08 87) (end 191.928 87) (width 0.2) (layer "F.Cu") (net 7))
 (segment (start 191.928 87) (end 191.928 87.2879) (width 0.2) (layer "F.Cu") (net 7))
 (segment (start 184.68 100.471) (end 183.217 99.0071) (width 0.2) (layer "F.Cu") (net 5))
 (segment (start 183.217 99.0071) (end 183.217 95.2375) (width 0.2) (layer "F.Cu") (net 5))
 (segment (start 183.604 94.85) (end 184.275 94.85) (width 0.2) (layer "F.Cu") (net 5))
 (segment (start 183.217 95.2375) (end 183.604 94.85) (width 0.2) (layer "F.Cu") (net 5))
 (segment (start 188.746 100.471) (end 184.68 100.471) (width 0.2) (layer "F.Cu") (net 5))
 (segment (start 189.775 101.5) (end 188.746 100.471) (width 0.2) (layer "F.Cu") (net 5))
 (segment (start 185.515 113.152) (end 191.648 113.152) (width 0.2) (layer "B.Cu") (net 1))
 (segment (start 191.648 113.152) (end 192.432 112.368) (width 0.2) (layer "B.Cu") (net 1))
 (segment (start 192.4325 109.4575) (end 192.4325 104.6825) (width 0.2) (layer "B.Cu") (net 1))
 (segment (start 192.432 109.458) (end 192.432 107.866) (width 0.2) (layer "B.Cu") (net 1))
 (segment (start 184.652 112) (end 184.652 112.288) (width 0.2) (layer "B.Cu") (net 1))
 (segment (start 184.652 112.288) (end 185.515 113.152) (width 0.2) (layer "B.Cu") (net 1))
 (segment (start 192.432 109.458) (end 192.4325 109.4575) (width 0.2) (layer "B.Cu") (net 1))
 (segment (start 183.5 112) (end 184.652 112) (width 0.2) (layer "B.Cu") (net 1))
 (segment (start 192.432 112.368) (end 192.432 109.458) (width 0.2) (layer "B.Cu") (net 1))
 (segment (start 184.275 92.9) (end 184.575736 92.599264) (width 0.2) (layer "F.Cu") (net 6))
 (segment (start 184.575736 92.599264) (end 184.575736 92.5) (width 0.2) (layer "F.Cu") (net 6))
 (segment (start 189 91.5) (end 187 93.5) (width 0.2) (layer "F.Cu") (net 6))
 (segment (start 193.5 91.5) (end 189 91.5) (width 0.2) (layer "F.Cu") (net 6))
 (segment (start 195.325 89.675) (end 193.5 91.5) (width 0.2) (layer "F.Cu") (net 6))
 (segment (start 184.575736 91.924264) (end 185 91.5) (width 0.2) (layer "F.Cu") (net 6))
 (segment (start 197.5 89.675) (end 195.325 89.675) (width 0.2) (layer "F.Cu") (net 6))
 (segment (start 184.575736 92.5) (end 184.575736 91.924264) (width 0.2) (layer "F.Cu") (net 6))
 (segment (start 184.575736 92.5) (end 184.575736 92.424264) (width 0.2) (layer "F.Cu") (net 6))
 (segment (start 187 93.5) (end 187 94) (width 0.2) (layer "F.Cu") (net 6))
 (via (at 187 94) (size 0.6) (drill 0.3) (layers "F.Cu" "B.Cu") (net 6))
 (via (at 185 91.5) (size 0.6) (drill 0.3) (layers "F.Cu" "B.Cu") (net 6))
 (segment (start 185 91.5) (end 185 92) (width 0.2) (layer "B.Cu") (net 6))
 (segment (start 185 92) (end 187 94) (width 0.2) (layer "B.Cu") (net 6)))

